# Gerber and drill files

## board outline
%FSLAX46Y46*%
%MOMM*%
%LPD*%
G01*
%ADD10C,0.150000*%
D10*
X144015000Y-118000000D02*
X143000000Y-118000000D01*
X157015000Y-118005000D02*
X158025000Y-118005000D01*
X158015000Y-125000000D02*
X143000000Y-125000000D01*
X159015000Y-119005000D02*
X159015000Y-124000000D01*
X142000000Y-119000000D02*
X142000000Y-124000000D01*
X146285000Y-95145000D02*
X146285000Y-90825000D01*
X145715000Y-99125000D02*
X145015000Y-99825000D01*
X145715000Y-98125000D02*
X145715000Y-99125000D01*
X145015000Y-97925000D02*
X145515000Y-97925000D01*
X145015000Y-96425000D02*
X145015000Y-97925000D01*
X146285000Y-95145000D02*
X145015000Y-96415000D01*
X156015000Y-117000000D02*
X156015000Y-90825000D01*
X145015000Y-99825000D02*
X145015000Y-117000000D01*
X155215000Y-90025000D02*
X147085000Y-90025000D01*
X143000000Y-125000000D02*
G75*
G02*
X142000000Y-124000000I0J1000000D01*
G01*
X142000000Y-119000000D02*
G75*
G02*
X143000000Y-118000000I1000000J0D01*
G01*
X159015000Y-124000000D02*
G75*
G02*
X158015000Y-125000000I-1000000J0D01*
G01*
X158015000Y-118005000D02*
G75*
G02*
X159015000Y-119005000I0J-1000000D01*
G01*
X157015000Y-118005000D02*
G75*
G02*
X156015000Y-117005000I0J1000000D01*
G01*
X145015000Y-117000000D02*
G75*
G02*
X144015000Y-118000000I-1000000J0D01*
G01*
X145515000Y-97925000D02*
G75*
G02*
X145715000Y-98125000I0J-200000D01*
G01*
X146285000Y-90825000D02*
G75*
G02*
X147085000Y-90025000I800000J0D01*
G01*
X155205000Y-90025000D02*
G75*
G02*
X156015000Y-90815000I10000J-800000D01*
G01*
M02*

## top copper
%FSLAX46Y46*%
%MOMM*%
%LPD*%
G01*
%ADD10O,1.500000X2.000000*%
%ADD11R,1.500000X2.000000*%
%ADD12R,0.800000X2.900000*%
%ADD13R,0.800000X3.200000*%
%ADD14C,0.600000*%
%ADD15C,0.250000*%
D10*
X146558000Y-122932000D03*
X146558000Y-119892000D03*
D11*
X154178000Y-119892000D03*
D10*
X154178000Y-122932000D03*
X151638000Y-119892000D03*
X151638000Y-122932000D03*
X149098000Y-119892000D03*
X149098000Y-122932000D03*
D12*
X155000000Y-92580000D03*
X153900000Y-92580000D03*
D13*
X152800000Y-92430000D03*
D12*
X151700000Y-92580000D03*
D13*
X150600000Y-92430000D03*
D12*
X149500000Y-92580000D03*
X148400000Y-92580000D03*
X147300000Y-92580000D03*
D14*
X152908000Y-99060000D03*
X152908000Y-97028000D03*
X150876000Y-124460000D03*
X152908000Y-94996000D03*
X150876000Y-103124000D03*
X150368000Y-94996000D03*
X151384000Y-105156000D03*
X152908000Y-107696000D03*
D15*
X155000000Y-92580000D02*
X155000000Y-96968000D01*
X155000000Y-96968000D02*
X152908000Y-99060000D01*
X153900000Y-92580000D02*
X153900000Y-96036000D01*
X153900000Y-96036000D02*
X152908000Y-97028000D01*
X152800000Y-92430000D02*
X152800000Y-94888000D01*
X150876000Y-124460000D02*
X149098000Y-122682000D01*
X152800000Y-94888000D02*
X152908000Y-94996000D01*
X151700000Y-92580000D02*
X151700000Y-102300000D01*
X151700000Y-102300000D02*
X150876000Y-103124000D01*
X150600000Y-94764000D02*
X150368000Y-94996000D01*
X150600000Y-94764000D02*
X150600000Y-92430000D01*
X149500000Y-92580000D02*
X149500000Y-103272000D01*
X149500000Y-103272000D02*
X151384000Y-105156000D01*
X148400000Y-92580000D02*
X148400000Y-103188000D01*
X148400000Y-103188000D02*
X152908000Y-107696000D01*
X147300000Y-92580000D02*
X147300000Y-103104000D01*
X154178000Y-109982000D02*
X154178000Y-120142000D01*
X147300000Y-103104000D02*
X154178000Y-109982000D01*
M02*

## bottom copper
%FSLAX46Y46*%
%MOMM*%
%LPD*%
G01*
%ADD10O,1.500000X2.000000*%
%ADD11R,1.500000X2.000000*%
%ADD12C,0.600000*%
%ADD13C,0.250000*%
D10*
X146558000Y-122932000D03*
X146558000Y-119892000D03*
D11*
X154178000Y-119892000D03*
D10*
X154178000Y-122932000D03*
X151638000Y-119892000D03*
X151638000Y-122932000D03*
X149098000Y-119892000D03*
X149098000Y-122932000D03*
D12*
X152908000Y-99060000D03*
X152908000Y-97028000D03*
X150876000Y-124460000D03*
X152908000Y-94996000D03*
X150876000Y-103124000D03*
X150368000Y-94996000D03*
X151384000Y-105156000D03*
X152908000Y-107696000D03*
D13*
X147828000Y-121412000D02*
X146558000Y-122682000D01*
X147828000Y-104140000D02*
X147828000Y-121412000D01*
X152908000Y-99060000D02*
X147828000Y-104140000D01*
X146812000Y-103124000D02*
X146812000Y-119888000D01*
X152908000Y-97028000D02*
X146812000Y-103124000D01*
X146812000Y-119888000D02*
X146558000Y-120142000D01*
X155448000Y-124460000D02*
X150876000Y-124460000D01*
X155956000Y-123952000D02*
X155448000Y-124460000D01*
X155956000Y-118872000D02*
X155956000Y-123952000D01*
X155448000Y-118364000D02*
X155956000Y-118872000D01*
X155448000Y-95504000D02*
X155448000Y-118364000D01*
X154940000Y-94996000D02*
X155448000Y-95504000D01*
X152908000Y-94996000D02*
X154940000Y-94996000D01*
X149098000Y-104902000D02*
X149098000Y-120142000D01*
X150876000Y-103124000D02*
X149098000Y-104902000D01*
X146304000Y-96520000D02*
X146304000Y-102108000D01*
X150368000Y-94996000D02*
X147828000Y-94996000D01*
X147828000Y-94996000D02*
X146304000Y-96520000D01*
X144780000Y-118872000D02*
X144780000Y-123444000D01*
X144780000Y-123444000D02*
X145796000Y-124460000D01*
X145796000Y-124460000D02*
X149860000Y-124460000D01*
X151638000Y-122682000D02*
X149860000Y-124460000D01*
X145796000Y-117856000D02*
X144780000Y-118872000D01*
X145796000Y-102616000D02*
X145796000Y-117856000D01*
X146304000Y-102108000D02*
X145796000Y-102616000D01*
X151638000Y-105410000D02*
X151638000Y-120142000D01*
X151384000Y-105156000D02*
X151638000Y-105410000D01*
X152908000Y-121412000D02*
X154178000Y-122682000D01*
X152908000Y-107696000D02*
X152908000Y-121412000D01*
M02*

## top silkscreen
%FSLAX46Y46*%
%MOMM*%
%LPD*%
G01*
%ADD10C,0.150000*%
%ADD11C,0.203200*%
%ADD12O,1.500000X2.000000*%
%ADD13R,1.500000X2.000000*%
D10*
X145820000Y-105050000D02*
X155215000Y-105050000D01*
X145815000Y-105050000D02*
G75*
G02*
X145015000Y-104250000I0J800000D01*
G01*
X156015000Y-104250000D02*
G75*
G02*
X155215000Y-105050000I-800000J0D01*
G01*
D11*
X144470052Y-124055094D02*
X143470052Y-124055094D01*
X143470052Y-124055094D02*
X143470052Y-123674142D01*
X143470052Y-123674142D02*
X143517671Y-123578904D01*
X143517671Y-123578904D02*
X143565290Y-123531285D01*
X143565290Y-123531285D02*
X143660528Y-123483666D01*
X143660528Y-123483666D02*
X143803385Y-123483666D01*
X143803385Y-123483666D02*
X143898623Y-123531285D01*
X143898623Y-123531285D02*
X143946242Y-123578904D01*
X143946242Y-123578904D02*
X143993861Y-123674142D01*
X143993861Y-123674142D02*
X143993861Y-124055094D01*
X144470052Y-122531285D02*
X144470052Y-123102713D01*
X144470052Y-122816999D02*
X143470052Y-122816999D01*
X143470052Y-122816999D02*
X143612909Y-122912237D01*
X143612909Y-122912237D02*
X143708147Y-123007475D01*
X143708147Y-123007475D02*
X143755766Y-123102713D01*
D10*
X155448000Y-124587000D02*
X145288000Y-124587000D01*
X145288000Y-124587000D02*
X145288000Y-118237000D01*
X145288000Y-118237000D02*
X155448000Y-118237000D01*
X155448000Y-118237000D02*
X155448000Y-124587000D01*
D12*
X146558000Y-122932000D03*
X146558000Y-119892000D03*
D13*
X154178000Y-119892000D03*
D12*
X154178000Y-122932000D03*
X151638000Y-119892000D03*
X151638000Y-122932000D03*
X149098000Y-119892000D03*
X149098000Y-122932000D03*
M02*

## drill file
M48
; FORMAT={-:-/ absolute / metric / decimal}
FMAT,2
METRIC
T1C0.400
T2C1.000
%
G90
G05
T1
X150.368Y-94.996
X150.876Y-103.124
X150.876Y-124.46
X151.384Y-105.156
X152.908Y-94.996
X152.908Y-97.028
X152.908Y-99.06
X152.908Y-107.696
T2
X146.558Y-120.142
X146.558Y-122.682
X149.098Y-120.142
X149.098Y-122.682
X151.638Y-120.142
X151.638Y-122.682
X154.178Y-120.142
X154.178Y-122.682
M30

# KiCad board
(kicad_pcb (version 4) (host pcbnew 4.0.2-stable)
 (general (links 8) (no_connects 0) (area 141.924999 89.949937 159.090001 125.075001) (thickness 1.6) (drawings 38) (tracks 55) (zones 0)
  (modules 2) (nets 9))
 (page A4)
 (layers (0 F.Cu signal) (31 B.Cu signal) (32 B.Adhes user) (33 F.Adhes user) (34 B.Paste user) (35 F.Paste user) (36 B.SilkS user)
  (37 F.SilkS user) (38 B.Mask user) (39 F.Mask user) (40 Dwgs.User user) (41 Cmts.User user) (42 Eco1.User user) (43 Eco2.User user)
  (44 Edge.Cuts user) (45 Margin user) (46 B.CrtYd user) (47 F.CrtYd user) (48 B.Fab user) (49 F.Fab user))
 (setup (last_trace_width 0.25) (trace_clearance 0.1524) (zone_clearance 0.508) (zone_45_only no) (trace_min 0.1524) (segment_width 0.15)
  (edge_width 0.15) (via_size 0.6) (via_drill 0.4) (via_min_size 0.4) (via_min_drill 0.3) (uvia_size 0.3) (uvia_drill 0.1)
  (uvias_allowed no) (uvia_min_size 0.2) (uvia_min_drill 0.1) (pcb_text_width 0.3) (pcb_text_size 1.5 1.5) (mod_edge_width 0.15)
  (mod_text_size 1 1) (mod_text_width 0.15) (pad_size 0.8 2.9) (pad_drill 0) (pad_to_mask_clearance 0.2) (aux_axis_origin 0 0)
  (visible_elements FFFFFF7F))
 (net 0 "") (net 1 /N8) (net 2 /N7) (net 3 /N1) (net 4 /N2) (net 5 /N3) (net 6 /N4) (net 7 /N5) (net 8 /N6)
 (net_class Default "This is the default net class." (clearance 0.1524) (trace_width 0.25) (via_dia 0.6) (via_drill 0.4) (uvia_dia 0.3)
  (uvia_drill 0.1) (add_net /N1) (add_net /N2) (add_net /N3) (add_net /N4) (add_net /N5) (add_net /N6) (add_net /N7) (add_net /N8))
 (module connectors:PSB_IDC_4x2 (layer F.Cu) (at 150.368 121.412 180)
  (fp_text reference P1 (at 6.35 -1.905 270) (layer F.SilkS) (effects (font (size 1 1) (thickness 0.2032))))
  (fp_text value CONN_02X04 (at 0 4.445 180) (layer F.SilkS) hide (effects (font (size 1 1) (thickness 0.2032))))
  (fp_line (start -5.08 -3.175) (end 5.08 -3.175) (layer F.SilkS) (width 0.15))
  (fp_line (start 5.08 -3.175) (end 5.08 3.175) (layer F.SilkS) (width 0.15))
  (fp_line (start 5.08 3.175) (end -5.08 3.175) (layer F.SilkS) (width 0.15))
  (fp_line (start -5.08 3.175) (end -5.08 -3.175) (layer F.SilkS) (width 0.15))
  (pad 8 thru_hole oval (at 3.81 -1.27 180) (size 1.5 2) (drill 1 (offset 0 -0.25)) (layers *.Cu *.Mask F.SilkS) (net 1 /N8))
  (pad 7 thru_hole oval (at 3.81 1.27 180) (size 1.5 2) (drill 1 (offset 0 0.25)) (layers *.Cu *.Mask F.SilkS) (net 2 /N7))
  (pad 1 thru_hole rect (at -3.81 1.27 180) (size 1.5 2) (drill 1 (offset 0 0.25)) (layers *.Cu *.Mask F.SilkS) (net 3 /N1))
  (pad 2 thru_hole oval (at -3.81 -1.27 180) (size 1.5 2) (drill 1 (offset 0 -0.25)) (layers *.Cu *.Mask F.SilkS) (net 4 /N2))
  (pad 3 thru_hole oval (at -1.27 1.27 180) (size 1.5 2) (drill 1 (offset 0 0.25)) (layers *.Cu *.Mask F.SilkS) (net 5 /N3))
  (pad 4 thru_hole oval (at -1.27 -1.27 180) (size 1.5 2) (drill 1 (offset 0 -0.25)) (layers *.Cu *.Mask F.SilkS) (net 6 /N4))
  (pad 5 thru_hole oval (at 1.27 1.27 180) (size 1.5 2) (drill 1 (offset 0 0.25)) (layers *.Cu *.Mask F.SilkS) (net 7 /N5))
  (pad 6 thru_hole oval (at 1.27 -1.27 180) (size 1.5 2) (drill 1 (offset 0 -0.25)) (layers *.Cu *.Mask F.SilkS) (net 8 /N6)))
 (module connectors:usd (layer F.Cu) (at 147.3 92.58)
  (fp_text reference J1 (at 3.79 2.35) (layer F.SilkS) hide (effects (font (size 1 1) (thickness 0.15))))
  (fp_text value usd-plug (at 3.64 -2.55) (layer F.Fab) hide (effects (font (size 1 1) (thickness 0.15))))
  (pad 8 smd rect (at 7.7 0) (size 0.8 2.9) (layers F.Cu F.Paste F.Mask) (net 1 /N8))
  (pad 7 smd rect (at 6.6 0) (size 0.8 2.9) (layers F.Cu F.Paste F.Mask) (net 2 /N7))
  (pad 6 smd rect (at 5.5 -0.15) (size 0.8 3.2) (layers F.Cu F.Paste F.Mask) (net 8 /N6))
  (pad 5 smd rect (at 4.4 0) (size 0.8 2.9) (layers F.Cu F.Paste F.Mask) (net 7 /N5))
  (pad 4 smd rect (at 3.3 -0.15) (size 0.8 3.2) (layers F.Cu F.Paste F.Mask) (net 6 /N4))
  (pad 3 smd rect (at 2.2 0) (size 0.8 2.9) (layers F.Cu F.Paste F.Mask) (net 5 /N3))
  (pad 2 smd rect (at 1.1 0) (size 0.8 2.9) (layers F.Cu F.Paste F.Mask) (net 4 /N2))
  (pad 1 smd rect (at 0 0) (size 0.8 2.9) (layers F.Cu F.Paste F.Mask) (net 3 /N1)))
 (gr_line (start 144.015 118) (end 143 118) (angle 90) (layer Edge.Cuts) (width 0.15))
 (gr_line (start 157.015 118.005) (end 158.025 118.005) (angle 90) (layer Edge.Cuts) (width 0.15))
 (gr_line (start 158.015 125) (end 143 125) (angle 90) (layer Edge.Cuts) (width 0.15))
 (gr_line (start 159.015 119.005) (end 159.015 124) (angle 90) (layer Edge.Cuts) (width 0.15))
 (gr_line (start 142 119) (end 142 124) (angle 90) (layer Edge.Cuts) (width 0.15))
 (gr_line (start 145.82 105.05) (end 155.215 105.05) (angle 90) (layer F.SilkS) (width 0.15))
 (gr_line (start 146.285 95.145) (end 146.285 90.825) (angle 90) (layer Edge.Cuts) (width 0.15))
 (gr_line (start 145.715 99.125) (end 145.015 99.825) (angle 90) (layer Edge.Cuts) (width 0.15))
 (gr_line (start 145.715 98.125) (end 145.715 99.125) (angle 90) (layer Edge.Cuts) (width 0.15))
 (gr_line (start 145.015 97.925) (end 145.515 97.925) (angle 90) (layer Edge.Cuts) (width 0.15))
 (gr_line (start 145.015 96.425) (end 145.015 97.925) (angle 90) (layer Edge.Cuts) (width 0.15))
 (gr_line (start 146.285 95.145) (end 145.015 96.415) (angle 90) (layer Edge.Cuts) (width 0.15))
 (gr_line (start 156.015 117) (end 156.015 90.825) (angle 90) (layer Edge.Cuts) (width 0.15))
 (gr_line (start 145.015 99.825) (end 145.015 117) (angle 90) (layer Edge.Cuts) (width 0.15))
 (gr_line (start 155.215 90.025) (end 147.085 90.025) (angle 90) (layer Edge.Cuts) (width 0.15))
 (gr_arc (start 143 124) (end 143 125) (angle 90) (layer Edge.Cuts) (width 0.15))
 (gr_arc (start 143 119) (end 142 119) (angle 90) (layer Edge.Cuts) (width 0.15))
 (gr_arc (start 158.015 124) (end 159.015 124) (angle 90) (layer Edge.Cuts) (width 0.15))
 (gr_arc (start 158.015 119.005) (end 158.015 118.005) (angle 90) (layer Edge.Cuts) (width 0.15))
 (gr_arc (start 157.015 117.005) (end 157.015 118.005) (angle 90) (layer Edge.Cuts) (width 0.15))
 (gr_arc (start 144.015 117) (end 145.015 117) (angle 90) (layer Edge.Cuts) (width 0.15))
 (gr_arc (start 145.815 104.25) (end 145.815 105.05) (angle 90) (layer F.SilkS) (width 0.15))
 (gr_arc (start 155.215 104.25) (end 156.015 104.25) (angle 90) (layer F.SilkS) (width 0.15))
 (gr_arc (start 145.515 98.125) (end 145.715 98.125) (angle -90) (layer Edge.Cuts) (width 0.15))
 (gr_arc (start 147.085 90.825) (end 147.085 90.025) (angle -90) (layer Edge.Cuts) (width 0.15))
 (gr_arc (start 155.215 90.825) (end 156.015 90.815) (angle -90) (layer Edge.Cuts) (width 0.15))
 (segment (start 155 92.58) (end 155 96.968) (width 0.25) (layer F.Cu) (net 1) (status 400000))
 (segment (start 147.828 121.412) (end 146.558 122.682) (width 0.25) (layer B.Cu) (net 1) (status 800000))
 (segment (start 147.828 104.14) (end 147.828 121.412) (width 0.25) (layer B.Cu) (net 1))
 (segment (start 152.908 99.06) (end 147.828 104.14) (width 0.25) (layer B.Cu) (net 1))
 (segment (start 155 96.968) (end 152.908 99.06) (width 0.25) (layer F.Cu) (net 1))
 (segment (start 153.9 92.58) (end 153.9 96.036) (width 0.25) (layer F.Cu) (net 2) (status 400000))
 (segment (start 146.812 103.124) (end 146.812 119.888) (width 0.25) (layer B.Cu) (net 2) (status 800000))
 (segment (start 152.908 97.028) (end 146.812 103.124) (width 0.25) (layer B.Cu) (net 2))
 (segment (start 153.9 96.036) (end 152.908 97.028) (width 0.25) (layer F.Cu) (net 2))
 (segment (start 146.812 119.888) (end 146.558 120.142) (width 0.25) (layer B.Cu) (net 2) (status C00000))
 (segment (start 152.8 92.43) (end 152.8 94.888) (width 0.25) (layer F.Cu) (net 8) (status 400000))
 (segment (start 150.876 124.46) (end 149.098 122.682) (width 0.25) (layer F.Cu) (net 8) (status 800000))
 (segment (start 155.448 124.46) (end 150.876 124.46) (width 0.25) (layer B.Cu) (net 8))
 (segment (start 155.956 123.952) (end 155.448 124.46) (width 0.25) (layer B.Cu) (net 8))
 (segment (start 155.956 118.872) (end 155.956 123.952) (width 0.25) (layer B.Cu) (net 8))
 (segment (start 155.448 118.364) (end 155.956 118.872) (width 0.25) (layer B.Cu) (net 8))
 (segment (start 155.448 95.504) (end 155.448 118.364) (width 0.25) (layer B.Cu) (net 8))
 (segment (start 154.94 94.996) (end 155.448 95.504) (width 0.25) (layer B.Cu) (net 8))
 (segment (start 152.908 94.996) (end 154.94 94.996) (width 0.25) (layer B.Cu) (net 8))
 (segment (start 152.8 94.888) (end 152.908 94.996) (width 0.25) (layer F.Cu) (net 8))
 (segment (start 151.7 92.58) (end 151.7 102.3) (width 0.25) (layer F.Cu) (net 7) (status 400000))
 (segment (start 149.098 104.902) (end 149.098 120.142) (width 0.25) (layer B.Cu) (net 7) (status 800000))
 (segment (start 150.876 103.124) (end 149.098 104.902) (width 0.25) (layer B.Cu) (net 7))
 (segment (start 151.7 102.3) (end 150.876 103.124) (width 0.25) (layer F.Cu) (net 7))
 (segment (start 146.304 96.52) (end 146.304 102.108) (width 0.25) (layer B.Cu) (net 6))
 (segment (start 150.6 94.764) (end 150.368 94.996) (width 0.25) (layer F.Cu) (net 6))
 (segment (start 150.368 94.996) (end 147.828 94.996) (width 0.25) (layer B.Cu) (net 6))
 (segment (start 147.828 94.996) (end 146.304 96.52) (width 0.25) (layer B.Cu) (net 6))
 (segment (start 144.78 118.872) (end 144.78 123.444) (width 0.25) (layer B.Cu) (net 6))
 (segment (start 144.78 123.444) (end 145.796 124.46) (width 0.25) (layer B.Cu) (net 6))
 (segment (start 145.796 124.46) (end 149.86 124.46) (width 0.25) (layer B.Cu) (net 6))
 (segment (start 151.638 122.682) (end 149.86 124.46) (width 0.25) (layer B.Cu) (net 6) (status 400000))
 (segment (start 150.6 94.764) (end 150.6 92.43) (width 0.25) (layer F.Cu) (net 6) (status 800000))
 (segment (start 145.796 117.856) (end 144.78 118.872) (width 0.25) (layer B.Cu) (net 6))
 (segment (start 145.796 102.616) (end 145.796 117.856) (width 0.25) (layer B.Cu) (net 6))
 (segment (start 146.304 102.108) (end 145.796 102.616) (width 0.25) (layer B.Cu) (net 6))
 (segment (start 149.5 92.58) (end 149.5 103.272) (width 0.25) (layer F.Cu) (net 5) (status 400000))
 (segment (start 151.638 105.41) (end 151.638 120.142) (width 0.25) (layer B.Cu) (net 5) (status 800000))
 (segment (start 151.384 105.156) (end 151.638 105.41) (width 0.25) (layer B.Cu) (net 5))
 (segment (start 149.5 103.272) (end 151.384 105.156) (width 0.25) (layer F.Cu) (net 5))
 (segment (start 148.4 92.58) (end 148.4 103.188) (width 0.25) (layer F.Cu) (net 4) (status 400000))
 (segment (start 152.908 121.412) (end 154.178 122.682) (width 0.25) (layer B.Cu) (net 4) (status 800000))
 (segment (start 152.908 107.696) (end 152.908 121.412) (width 0.25) (layer B.Cu) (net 4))
 (segment (start 148.4 103.188) (end 152.908 107.696) (width 0.25) (layer F.Cu) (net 4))
 (segment (start 147.3 92.58) (end 147.3 103.104) (width 0.25) (layer F.Cu) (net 3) (status 400000))
 (segment (start 154.178 109.982) (end 154.178 120.142) (width 0.25) (layer F.Cu) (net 3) (status 800000))
 (segment (start 147.3 103.104) (end 154.178 109.982) (width 0.25) (layer F.Cu) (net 3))
 (via (at 152.908 99.06) (size 0.6) (drill 0.4) (layers F.Cu B.Cu) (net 1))
 (via (at 152.908 97.028) (size 0.6) (drill 0.4) (layers F.Cu B.Cu) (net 2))
 (via (at 150.876 124.46) (size 0.6) (drill 0.4) (layers F.Cu B.Cu) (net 8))
 (via (at 152.908 94.996) (size 0.6) (drill 0.4) (layers F.Cu B.Cu) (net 8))
 (via (at 150.876 103.124) (size 0.6) (drill 0.4) (layers F.Cu B.Cu) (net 7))
 (via (at 150.368 94.996) (size 0.6) (drill 0.4) (layers F.Cu B.Cu) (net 6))
 (via (at 151.384 105.156) (size 0.6) (drill 0.4) (layers F.Cu B.Cu) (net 5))
 (via (at 152.908 107.696) (size 0.6) (drill 0.4) (layers F.Cu B.Cu) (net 4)))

